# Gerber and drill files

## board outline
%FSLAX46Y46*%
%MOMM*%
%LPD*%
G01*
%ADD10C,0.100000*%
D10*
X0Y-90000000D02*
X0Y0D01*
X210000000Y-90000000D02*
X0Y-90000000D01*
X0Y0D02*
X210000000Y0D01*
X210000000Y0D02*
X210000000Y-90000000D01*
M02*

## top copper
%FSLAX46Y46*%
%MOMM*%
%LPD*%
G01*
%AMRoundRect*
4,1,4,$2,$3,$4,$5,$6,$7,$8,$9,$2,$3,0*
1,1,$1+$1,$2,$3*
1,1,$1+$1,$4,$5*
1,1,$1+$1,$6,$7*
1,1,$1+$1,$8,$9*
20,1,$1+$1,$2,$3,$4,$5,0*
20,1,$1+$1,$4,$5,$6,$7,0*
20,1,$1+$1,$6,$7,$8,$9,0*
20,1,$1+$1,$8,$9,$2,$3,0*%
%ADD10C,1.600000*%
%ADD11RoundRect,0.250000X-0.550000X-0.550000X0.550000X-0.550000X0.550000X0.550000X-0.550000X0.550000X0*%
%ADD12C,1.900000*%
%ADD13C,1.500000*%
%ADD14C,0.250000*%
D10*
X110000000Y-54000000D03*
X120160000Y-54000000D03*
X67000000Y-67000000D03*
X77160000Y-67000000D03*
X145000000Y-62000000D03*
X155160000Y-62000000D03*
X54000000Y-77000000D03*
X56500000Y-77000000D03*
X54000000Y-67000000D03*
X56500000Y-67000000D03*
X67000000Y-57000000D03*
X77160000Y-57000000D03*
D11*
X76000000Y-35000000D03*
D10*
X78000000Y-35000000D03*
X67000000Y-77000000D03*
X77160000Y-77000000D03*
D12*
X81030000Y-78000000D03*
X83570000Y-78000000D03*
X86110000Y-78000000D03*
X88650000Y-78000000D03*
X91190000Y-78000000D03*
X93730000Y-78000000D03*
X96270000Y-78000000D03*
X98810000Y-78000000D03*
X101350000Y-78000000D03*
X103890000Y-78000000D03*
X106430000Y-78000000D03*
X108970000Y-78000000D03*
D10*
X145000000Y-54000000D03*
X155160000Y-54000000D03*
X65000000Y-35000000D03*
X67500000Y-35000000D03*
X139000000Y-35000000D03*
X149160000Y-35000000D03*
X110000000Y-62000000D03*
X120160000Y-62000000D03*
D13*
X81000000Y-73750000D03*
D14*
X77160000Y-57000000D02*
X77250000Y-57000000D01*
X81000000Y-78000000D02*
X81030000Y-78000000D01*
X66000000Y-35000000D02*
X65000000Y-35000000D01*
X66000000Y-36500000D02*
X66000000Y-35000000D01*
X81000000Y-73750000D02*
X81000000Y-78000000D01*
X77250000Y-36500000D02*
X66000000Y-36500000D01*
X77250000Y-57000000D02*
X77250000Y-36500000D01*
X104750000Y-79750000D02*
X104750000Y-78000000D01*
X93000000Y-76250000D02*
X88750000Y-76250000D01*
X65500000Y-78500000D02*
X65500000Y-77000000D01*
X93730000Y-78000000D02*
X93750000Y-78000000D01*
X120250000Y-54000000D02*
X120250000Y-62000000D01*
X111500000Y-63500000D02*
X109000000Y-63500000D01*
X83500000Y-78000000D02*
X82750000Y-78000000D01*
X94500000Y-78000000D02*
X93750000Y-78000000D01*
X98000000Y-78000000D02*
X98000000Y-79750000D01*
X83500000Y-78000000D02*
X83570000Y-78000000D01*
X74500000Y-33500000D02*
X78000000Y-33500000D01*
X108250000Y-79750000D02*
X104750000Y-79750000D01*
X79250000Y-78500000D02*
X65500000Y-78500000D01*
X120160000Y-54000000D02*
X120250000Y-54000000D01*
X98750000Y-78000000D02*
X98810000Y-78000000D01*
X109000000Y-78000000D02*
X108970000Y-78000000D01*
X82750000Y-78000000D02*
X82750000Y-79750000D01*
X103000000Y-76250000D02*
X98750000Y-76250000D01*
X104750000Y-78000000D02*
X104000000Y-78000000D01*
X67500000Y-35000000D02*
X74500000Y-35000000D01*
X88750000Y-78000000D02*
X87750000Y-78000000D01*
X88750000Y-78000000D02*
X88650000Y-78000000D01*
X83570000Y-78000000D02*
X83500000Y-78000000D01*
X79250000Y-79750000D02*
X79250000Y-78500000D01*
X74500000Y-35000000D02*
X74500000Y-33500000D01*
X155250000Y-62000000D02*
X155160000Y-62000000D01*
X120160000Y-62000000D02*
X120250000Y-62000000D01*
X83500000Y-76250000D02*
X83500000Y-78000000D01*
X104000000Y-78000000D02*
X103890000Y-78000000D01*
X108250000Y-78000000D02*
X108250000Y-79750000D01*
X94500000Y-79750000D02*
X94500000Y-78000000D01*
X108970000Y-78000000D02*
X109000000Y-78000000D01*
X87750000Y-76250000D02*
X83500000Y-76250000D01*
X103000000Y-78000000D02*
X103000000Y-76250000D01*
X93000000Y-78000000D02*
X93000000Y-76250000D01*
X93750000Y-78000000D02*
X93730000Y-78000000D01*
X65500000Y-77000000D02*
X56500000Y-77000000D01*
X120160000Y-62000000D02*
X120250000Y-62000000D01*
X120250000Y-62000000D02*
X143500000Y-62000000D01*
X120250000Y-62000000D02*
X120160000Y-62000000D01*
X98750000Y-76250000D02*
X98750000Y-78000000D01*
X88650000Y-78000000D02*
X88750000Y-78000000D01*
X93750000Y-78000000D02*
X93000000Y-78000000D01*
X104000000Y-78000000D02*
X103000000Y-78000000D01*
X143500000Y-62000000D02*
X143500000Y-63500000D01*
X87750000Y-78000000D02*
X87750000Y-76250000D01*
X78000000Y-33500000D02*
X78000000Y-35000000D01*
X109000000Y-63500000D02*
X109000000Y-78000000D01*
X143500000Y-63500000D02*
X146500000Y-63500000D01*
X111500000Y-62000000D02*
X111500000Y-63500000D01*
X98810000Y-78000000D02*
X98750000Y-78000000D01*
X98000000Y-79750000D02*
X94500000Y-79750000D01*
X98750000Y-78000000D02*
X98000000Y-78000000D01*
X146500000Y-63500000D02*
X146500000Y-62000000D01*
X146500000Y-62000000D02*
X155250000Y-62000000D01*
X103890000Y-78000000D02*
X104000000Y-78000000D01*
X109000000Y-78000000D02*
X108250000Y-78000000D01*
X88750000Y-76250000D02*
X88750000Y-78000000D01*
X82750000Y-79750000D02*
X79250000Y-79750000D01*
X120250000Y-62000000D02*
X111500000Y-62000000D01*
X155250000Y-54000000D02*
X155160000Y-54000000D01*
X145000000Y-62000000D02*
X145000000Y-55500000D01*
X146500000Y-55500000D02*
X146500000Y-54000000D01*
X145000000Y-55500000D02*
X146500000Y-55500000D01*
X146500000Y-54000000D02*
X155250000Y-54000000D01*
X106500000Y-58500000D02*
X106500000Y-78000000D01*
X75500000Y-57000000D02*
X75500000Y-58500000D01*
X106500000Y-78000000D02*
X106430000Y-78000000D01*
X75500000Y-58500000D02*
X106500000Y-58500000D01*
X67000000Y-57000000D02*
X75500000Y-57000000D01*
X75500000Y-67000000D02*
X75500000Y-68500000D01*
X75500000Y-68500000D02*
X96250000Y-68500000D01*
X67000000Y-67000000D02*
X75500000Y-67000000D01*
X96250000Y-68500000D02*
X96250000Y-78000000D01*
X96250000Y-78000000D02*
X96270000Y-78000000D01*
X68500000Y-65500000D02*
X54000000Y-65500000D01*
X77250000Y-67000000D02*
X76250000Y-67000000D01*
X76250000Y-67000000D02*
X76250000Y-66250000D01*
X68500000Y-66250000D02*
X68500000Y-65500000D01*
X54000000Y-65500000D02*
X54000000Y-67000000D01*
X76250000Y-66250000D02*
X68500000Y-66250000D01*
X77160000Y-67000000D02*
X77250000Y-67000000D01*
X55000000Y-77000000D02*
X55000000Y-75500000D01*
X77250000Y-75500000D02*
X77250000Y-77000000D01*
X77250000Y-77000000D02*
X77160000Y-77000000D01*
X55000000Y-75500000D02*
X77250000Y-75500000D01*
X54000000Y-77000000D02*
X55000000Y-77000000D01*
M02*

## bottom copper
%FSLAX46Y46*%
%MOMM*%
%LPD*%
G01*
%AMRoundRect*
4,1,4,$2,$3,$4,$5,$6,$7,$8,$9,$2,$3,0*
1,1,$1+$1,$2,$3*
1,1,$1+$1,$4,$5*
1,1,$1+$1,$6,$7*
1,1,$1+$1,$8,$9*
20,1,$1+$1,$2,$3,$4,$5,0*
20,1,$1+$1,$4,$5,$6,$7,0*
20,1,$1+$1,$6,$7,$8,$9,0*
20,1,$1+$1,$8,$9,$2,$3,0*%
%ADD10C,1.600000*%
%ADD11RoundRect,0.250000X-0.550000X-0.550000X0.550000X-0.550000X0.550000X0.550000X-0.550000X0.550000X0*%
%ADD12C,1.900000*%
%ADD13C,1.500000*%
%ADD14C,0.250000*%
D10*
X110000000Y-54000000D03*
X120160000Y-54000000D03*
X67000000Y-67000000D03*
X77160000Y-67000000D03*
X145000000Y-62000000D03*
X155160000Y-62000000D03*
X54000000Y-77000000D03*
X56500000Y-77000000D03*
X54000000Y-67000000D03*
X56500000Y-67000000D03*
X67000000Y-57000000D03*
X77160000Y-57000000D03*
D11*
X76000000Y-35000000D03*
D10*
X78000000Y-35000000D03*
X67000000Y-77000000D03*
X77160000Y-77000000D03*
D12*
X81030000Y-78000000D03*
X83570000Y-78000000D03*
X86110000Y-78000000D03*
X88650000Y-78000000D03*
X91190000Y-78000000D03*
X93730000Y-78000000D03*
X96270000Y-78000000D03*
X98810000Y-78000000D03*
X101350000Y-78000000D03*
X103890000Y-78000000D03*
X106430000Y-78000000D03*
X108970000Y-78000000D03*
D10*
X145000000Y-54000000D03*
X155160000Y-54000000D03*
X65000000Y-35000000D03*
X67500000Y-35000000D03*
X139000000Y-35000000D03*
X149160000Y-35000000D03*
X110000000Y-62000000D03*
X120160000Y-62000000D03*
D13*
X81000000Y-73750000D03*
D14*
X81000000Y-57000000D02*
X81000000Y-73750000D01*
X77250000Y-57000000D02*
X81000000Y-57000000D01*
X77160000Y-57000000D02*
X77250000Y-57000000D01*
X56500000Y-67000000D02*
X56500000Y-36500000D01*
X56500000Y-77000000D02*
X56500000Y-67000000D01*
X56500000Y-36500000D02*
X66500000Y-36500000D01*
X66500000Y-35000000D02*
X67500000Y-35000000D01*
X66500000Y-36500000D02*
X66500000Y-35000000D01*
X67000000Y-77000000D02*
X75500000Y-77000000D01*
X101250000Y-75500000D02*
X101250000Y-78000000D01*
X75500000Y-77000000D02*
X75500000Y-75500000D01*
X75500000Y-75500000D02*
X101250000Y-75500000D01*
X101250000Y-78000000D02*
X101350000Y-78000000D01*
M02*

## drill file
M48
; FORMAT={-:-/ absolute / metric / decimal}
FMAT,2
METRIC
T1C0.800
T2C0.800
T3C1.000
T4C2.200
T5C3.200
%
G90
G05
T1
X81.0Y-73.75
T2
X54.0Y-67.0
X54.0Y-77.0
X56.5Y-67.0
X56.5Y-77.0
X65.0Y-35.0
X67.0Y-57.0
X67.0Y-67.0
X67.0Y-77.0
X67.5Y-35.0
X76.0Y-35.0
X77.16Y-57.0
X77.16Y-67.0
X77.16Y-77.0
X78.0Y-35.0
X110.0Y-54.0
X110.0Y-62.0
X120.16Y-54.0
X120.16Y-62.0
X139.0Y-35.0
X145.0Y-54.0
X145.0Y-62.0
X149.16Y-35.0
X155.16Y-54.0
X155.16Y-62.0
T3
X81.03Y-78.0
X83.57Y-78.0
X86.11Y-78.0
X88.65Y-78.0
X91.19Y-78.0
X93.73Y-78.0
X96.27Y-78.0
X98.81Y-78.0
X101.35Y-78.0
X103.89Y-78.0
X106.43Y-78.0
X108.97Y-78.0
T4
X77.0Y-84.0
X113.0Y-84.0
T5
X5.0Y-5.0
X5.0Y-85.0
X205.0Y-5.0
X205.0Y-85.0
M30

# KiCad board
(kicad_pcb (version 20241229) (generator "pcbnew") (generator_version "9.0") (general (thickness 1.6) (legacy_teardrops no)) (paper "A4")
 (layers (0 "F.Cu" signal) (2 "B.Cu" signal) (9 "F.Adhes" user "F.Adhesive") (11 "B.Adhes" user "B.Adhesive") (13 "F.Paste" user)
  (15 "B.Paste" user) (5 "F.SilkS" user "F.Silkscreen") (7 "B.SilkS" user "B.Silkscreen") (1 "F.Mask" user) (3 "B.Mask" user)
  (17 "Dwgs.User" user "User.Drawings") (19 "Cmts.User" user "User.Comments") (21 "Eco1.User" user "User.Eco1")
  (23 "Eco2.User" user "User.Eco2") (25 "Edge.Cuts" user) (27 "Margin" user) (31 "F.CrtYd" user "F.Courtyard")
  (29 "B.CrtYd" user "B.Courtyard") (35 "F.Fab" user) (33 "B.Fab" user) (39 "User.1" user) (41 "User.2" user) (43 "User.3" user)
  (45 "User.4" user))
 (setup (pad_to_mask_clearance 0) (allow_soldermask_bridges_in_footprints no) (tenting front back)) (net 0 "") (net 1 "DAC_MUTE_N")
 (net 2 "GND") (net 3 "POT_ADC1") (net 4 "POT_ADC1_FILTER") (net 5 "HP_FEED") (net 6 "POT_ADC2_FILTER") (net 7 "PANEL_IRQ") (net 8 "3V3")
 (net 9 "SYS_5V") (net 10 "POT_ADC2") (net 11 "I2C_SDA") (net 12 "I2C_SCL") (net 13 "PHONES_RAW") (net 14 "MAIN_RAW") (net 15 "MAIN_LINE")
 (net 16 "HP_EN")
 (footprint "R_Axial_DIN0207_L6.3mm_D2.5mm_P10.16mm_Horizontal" (layer "F.Cu") (at 110 54)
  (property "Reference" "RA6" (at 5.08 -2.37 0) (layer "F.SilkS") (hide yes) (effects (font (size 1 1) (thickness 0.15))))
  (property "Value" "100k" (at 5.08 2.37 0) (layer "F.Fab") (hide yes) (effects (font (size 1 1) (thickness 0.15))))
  (pad "1" thru_hole circle (at 0 0) (size 1.6 1.6) (drill 0.8) (layers "*.Cu" "*.Mask") (remove_unused_layers no) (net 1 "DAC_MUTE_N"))
  (pad "2" thru_hole circle (at 10.16 0) (size 1.6 1.6) (drill 0.8) (layers "*.Cu" "*.Mask") (remove_unused_layers no) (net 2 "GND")))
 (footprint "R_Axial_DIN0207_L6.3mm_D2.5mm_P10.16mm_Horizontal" (layer "F.Cu") (at 67 67)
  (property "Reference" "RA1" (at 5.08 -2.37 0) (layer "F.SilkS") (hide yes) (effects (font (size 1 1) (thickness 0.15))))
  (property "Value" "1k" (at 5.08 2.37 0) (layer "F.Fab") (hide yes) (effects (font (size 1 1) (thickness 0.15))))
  (pad "1" thru_hole circle (at 0 0) (size 1.6 1.6) (drill 0.8) (layers "*.Cu" "*.Mask") (remove_unused_layers no) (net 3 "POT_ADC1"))
  (pad "2" thru_hole circle (at 10.16 0) (size 1.6 1.6) (drill 0.8) (layers "*.Cu" "*.Mask") (remove_unused_layers no)
   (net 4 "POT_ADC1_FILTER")))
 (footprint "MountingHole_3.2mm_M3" (layer "F.Cu") (at 5 5)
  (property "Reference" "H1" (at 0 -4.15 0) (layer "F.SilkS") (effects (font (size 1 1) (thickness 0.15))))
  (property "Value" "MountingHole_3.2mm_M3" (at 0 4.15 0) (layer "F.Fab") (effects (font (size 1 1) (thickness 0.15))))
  (pad "" np_thru_hole circle (at 0 0) (size 3.2 3.2) (drill 3.2) (layers "*.Cu" "*.Mask")))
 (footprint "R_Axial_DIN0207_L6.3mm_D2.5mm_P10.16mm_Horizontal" (layer "F.Cu") (at 145 62)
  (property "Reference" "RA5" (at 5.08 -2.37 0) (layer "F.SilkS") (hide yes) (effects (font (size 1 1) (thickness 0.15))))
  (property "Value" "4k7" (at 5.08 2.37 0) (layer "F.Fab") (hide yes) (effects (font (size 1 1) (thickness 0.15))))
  (pad "1" thru_hole circle (at 0 0) (size 1.6 1.6) (drill 0.8) (layers "*.Cu" "*.Mask") (remove_unused_layers no) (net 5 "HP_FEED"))
  (pad "2" thru_hole circle (at 10.16 0) (size 1.6 1.6) (drill 0.8) (layers "*.Cu" "*.Mask") (remove_unused_layers no) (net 2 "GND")))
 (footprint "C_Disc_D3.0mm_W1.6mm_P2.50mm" (layer "F.Cu") (at 54 77)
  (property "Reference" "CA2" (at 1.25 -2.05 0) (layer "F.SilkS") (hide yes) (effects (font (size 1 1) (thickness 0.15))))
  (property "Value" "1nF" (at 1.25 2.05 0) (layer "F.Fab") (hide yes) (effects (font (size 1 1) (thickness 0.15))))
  (pad "1" thru_hole circle (at 0 0) (size 1.6 1.6) (drill 0.8) (layers "*.Cu" "*.Mask") (remove_unused_layers no) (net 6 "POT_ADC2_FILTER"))
  (pad "2" thru_hole circle (at 2.5 0) (size 1.6 1.6) (drill 0.8) (layers "*.Cu" "*.Mask") (remove_unused_layers no) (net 2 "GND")))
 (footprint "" (layer "F.Cu") (at 112 42)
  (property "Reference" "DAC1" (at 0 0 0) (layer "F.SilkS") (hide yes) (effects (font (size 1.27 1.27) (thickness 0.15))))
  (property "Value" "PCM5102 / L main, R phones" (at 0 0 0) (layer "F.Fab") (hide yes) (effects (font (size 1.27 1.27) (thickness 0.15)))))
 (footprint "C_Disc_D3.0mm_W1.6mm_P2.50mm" (layer "F.Cu") (at 54 67)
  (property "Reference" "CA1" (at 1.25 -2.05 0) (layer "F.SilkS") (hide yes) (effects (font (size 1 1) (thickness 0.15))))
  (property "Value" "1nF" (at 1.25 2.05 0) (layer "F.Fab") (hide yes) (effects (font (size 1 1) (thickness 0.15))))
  (pad "1" thru_hole circle (at 0 0) (size 1.6 1.6) (drill 0.8) (layers "*.Cu" "*.Mask") (remove_unused_layers no) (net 4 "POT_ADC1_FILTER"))
  (pad "2" thru_hole circle (at 2.5 0) (size 1.6 1.6) (drill 0.8) (layers "*.Cu" "*.Mask") (remove_unused_layers no) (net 2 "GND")))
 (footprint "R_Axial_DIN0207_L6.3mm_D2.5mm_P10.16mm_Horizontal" (layer "F.Cu") (at 67 57)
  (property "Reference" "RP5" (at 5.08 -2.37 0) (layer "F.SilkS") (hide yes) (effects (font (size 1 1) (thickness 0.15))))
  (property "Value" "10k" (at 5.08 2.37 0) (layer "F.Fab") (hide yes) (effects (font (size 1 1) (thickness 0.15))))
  (pad "1" thru_hole circle (at 0 0) (size 1.6 1.6) (drill 0.8) (layers "*.Cu" "*.Mask") (remove_unused_layers no) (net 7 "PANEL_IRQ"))
  (pad "2" thru_hole circle (at 10.16 0) (size 1.6 1.6) (drill 0.8) (layers "*.Cu" "*.Mask") (remove_unused_layers no) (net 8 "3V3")))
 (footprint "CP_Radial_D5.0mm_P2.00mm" (layer "F.Cu") (at 76 35)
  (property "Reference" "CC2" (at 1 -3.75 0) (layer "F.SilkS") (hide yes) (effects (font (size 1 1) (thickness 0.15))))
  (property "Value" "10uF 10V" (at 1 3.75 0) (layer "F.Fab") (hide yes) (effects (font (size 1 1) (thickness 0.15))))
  (pad "1" thru_hole roundrect (at 0 0) (size 1.6 1.6) (drill 0.8) (layers "*.Cu" "*.Mask") (remove_unused_layers no)
   (roundrect_rratio 0.15625) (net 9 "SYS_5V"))
  (pad "2" thru_hole circle (at 2 0) (size 1.6 1.6) (drill 0.8) (layers "*.Cu" "*.Mask") (remove_unused_layers no) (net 2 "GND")))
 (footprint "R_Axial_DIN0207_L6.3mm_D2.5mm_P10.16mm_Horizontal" (layer "F.Cu") (at 67 77)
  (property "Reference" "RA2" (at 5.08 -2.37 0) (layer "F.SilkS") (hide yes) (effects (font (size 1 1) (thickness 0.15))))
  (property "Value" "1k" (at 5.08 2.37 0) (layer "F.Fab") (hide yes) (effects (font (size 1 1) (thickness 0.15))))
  (pad "1" thru_hole circle (at 0 0) (size 1.6 1.6) (drill 0.8) (layers "*.Cu" "*.Mask") (remove_unused_layers no) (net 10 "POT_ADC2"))
  (pad "2" thru_hole circle (at 10.16 0) (size 1.6 1.6) (drill 0.8) (layers "*.Cu" "*.Mask") (remove_unused_layers no)
   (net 6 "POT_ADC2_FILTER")))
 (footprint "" (layer "F.Cu") (at 174 13)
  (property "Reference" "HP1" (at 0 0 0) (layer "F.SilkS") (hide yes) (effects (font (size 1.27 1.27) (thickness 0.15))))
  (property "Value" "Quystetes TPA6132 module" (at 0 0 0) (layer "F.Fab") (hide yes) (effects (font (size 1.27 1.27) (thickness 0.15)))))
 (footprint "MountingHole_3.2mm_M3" (layer "F.Cu") (at 205 5)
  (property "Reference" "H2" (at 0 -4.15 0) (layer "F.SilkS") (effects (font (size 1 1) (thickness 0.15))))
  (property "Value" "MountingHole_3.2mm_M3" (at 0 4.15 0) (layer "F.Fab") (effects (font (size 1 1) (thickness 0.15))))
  (pad "" np_thru_hole circle (at 0 0) (size 3.2 3.2) (drill 3.2) (layers "*.Cu" "*.Mask")))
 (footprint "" (layer "F.Cu") (at 95 78)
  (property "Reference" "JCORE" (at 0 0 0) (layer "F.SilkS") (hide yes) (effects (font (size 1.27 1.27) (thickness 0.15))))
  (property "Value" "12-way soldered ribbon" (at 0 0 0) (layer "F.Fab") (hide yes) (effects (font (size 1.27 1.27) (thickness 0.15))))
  (pad "1" thru_hole circle (at -13.97 0) (size 1.9 1.9) (drill 1) (layers "*.Cu") (remove_unused_layers no) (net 8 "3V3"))
  (pad "2" thru_hole circle (at -11.43 0) (size 1.9 1.9) (drill 1) (layers "*.Cu") (remove_unused_layers no) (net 2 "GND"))
  (pad "3" thru_hole circle (at -8.89 0) (size 1.9 1.9) (drill 1) (layers "*.Cu") (remove_unused_layers no) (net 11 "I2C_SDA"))
  (pad "4" thru_hole circle (at -6.35 0) (size 1.9 1.9) (drill 1) (layers "*.Cu") (remove_unused_layers no) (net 2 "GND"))
  (pad "5" thru_hole circle (at -3.81 0) (size 1.9 1.9) (drill 1) (layers "*.Cu") (remove_unused_layers no) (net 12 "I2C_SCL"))
  (pad "6" thru_hole circle (at -1.27 0) (size 1.9 1.9) (drill 1) (layers "*.Cu") (remove_unused_layers no) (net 2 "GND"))
  (pad "7" thru_hole circle (at 1.27 0) (size 1.9 1.9) (drill 1) (layers "*.Cu") (remove_unused_layers no) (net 3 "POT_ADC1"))
  (pad "8" thru_hole circle (at 3.81 0) (size 1.9 1.9) (drill 1) (layers "*.Cu") (remove_unused_layers no) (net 2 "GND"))
  (pad "9" thru_hole circle (at 6.35 0) (size 1.9 1.9) (drill 1) (layers "*.Cu") (remove_unused_layers no) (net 10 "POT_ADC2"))
  (pad "10" thru_hole circle (at 8.89 0) (size 1.9 1.9) (drill 1) (layers "*.Cu") (remove_unused_layers no) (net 2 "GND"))
  (pad "11" thru_hole circle (at 11.43 0) (size 1.9 1.9) (drill 1) (layers "*.Cu") (remove_unused_layers no) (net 7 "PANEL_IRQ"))
  (pad "12" thru_hole circle (at 13.97 0) (size 1.9 1.9) (drill 1) (layers "*.Cu") (remove_unused_layers no) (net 2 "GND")))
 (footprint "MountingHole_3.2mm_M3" (layer "F.Cu") (at 5 85)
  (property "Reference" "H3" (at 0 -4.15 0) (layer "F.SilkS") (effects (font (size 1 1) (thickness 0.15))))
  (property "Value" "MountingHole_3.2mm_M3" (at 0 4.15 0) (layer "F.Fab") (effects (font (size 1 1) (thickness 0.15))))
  (pad "" np_thru_hole circle (at 0 0) (size 3.2 3.2) (drill 3.2) (layers "*.Cu" "*.Mask")))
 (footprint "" (layer "F.Cu") (at 144 5)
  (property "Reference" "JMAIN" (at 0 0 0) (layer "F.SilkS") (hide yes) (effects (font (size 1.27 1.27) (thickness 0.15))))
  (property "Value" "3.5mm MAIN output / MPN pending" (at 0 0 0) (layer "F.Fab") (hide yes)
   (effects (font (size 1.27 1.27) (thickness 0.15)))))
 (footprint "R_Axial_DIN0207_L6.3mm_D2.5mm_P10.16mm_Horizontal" (layer "F.Cu") (at 145 54)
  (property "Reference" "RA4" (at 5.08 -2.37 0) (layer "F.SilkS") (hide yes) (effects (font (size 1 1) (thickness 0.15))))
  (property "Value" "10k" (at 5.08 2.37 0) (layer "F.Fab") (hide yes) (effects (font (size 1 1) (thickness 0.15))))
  (pad "1" thru_hole circle (at 0 0) (size 1.6 1.6) (drill 0.8) (layers "*.Cu" "*.Mask") (remove_unused_layers no) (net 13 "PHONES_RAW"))
  (pad "2" thru_hole circle (at 10.16 0) (size 1.6 1.6) (drill 0.8) (layers "*.Cu" "*.Mask") (remove_unused_layers no) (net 5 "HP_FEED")))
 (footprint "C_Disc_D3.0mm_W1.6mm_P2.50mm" (layer "F.Cu") (at 65 35)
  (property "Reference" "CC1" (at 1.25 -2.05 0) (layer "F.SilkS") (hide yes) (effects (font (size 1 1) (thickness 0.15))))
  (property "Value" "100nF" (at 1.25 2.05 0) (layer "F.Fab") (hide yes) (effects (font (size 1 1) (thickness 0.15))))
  (pad "1" thru_hole circle (at 0 0) (size 1.6 1.6) (drill 0.8) (layers "*.Cu" "*.Mask") (remove_unused_layers no) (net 8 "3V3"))
  (pad "2" thru_hole circle (at 2.5 0) (size 1.6 1.6) (drill 0.8) (layers "*.Cu" "*.Mask") (remove_unused_layers no) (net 2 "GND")))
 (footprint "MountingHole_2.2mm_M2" (layer "F.Cu") (at 77 84)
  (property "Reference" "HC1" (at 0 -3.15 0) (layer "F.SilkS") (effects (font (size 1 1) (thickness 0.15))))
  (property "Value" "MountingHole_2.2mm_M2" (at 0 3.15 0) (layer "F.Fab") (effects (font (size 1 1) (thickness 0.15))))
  (pad "" np_thru_hole circle (at 0 0) (size 2.2 2.2) (drill 2.2) (layers "*.Cu" "*.Mask")))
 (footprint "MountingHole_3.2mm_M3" (layer "F.Cu") (at 205 85)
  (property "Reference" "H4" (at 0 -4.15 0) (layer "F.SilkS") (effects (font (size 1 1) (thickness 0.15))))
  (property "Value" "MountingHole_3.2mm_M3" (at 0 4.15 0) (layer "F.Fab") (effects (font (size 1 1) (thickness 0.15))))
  (pad "" np_thru_hole circle (at 0 0) (size 3.2 3.2) (drill 3.2) (layers "*.Cu" "*.Mask")))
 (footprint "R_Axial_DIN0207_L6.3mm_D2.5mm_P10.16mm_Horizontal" (layer "F.Cu") (at 139 35)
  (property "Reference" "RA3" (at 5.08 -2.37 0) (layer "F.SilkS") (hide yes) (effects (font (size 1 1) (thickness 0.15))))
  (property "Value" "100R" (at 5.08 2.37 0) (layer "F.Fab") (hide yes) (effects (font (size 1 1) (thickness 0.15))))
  (pad "1" thru_hole circle (at 0 0) (size 1.6 1.6) (drill 0.8) (layers "*.Cu" "*.Mask") (remove_unused_layers no) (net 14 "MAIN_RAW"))
  (pad "2" thru_hole circle (at 10.16 0) (size 1.6 1.6) (drill 0.8) (layers "*.Cu" "*.Mask") (remove_unused_layers no) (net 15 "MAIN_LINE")))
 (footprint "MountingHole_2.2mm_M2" (layer "F.Cu") (at 113 84)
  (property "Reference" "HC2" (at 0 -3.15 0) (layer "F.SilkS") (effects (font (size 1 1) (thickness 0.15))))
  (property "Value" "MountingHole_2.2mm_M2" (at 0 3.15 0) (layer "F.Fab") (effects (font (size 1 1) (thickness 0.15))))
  (pad "" np_thru_hole circle (at 0 0) (size 2.2 2.2) (drill 2.2) (layers "*.Cu" "*.Mask")))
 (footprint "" (layer "F.Cu") (at 30 31)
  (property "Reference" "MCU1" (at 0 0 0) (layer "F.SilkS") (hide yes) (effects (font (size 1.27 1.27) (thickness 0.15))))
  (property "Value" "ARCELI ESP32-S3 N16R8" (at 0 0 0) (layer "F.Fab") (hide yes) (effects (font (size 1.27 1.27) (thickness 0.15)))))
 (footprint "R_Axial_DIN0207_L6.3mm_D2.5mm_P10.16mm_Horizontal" (layer "F.Cu") (at 110 62)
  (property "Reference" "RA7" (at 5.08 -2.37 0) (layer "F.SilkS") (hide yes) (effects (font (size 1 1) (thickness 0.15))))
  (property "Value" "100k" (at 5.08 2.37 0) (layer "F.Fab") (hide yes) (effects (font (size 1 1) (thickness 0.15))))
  (pad "1" thru_hole circle (at 0 0) (size 1.6 1.6) (drill 0.8) (layers "*.Cu" "*.Mask") (remove_unused_layers no) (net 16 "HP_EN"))
  (pad "2" thru_hole circle (at 10.16 0) (size 1.6 1.6) (drill 0.8) (layers "*.Cu" "*.Mask") (remove_unused_layers no) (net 2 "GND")))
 (gr_line (start 0 90) (end 0 0) (stroke (width 0.1) (type default)) (layer "Edge.Cuts"))
 (gr_line (start 210 90) (end 0 90) (stroke (width 0.1) (type default)) (layer "Edge.Cuts"))
 (gr_line (start 0 0) (end 210 0) (stroke (width 0.1) (type default)) (layer "Edge.Cuts"))
 (gr_line (start 210 0) (end 210 90) (stroke (width 0.1) (type default)) (layer "Edge.Cuts"))
 (segment (start 77.16 57) (end 77.25 57) (width 0.25) (layer "F.Cu") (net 8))
 (segment (start 81 78) (end 81.03 78) (width 0.25) (layer "F.Cu") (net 8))
 (segment (start 66 35) (end 65 35) (width 0.25) (layer "F.Cu") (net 8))
 (segment (start 66 36.5) (end 66 35) (width 0.25) (layer "F.Cu") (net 8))
 (segment (start 81 73.75) (end 81 78) (width 0.25) (layer "F.Cu") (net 8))
 (segment (start 77.25 36.5) (end 66 36.5) (width 0.25) (layer "F.Cu") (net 8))
 (segment (start 77.25 57) (end 77.25 36.5) (width 0.25) (layer "F.Cu") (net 8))
 (via (at 81 73.75) (size 1.5) (drill 0.8) (layers "F.Cu" "B.Cu") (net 8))
 (segment (start 81 57) (end 81 73.75) (width 0.25) (layer "B.Cu") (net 8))
 (segment (start 77.25 57) (end 81 57) (width 0.25) (layer "B.Cu") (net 8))
 (segment (start 77.16 57) (end 77.25 57) (width 0.25) (layer "B.Cu") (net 8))
 (segment (start 104.75 79.75) (end 104.75 78) (width 0.25) (layer "F.Cu") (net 2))
 (segment (start 93 76.25) (end 88.75 76.25) (width 0.25) (layer "F.Cu") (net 2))
 (segment (start 65.5 78.5) (end 65.5 77) (width 0.25) (layer "F.Cu") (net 2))
 (segment (start 93.73 78) (end 93.75 78) (width 0.25) (layer "F.Cu") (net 2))
 (segment (start 120.25 54) (end 120.25 62) (width 0.25) (layer "F.Cu") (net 2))
 (segment (start 111.5 63.5) (end 109 63.5) (width 0.25) (layer "F.Cu") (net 2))
 (segment (start 83.5 78) (end 82.75 78) (width 0.25) (layer "F.Cu") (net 2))
 (segment (start 94.5 78) (end 93.75 78) (width 0.25) (layer "F.Cu") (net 2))
 (segment (start 98 78) (end 98 79.75) (width 0.25) (layer "F.Cu") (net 2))
 (segment (start 83.5 78) (end 83.57 78) (width 0.25) (layer "F.Cu") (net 2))
 (segment (start 74.5 33.5) (end 78 33.5) (width 0.25) (layer "F.Cu") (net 2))
 (segment (start 108.25 79.75) (end 104.75 79.75) (width 0.25) (layer "F.Cu") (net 2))
 (segment (start 79.25 78.5) (end 65.5 78.5) (width 0.25) (layer "F.Cu") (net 2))
 (segment (start 120.16 54) (end 120.25 54) (width 0.25) (layer "F.Cu") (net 2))
 (segment (start 98.75 78) (end 98.81 78) (width 0.25) (layer "F.Cu") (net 2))
 (segment (start 109 78) (end 108.97 78) (width 0.25) (layer "F.Cu") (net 2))
 (segment (start 82.75 78) (end 82.75 79.75) (width 0.25) (layer "F.Cu") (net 2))
 (segment (start 103 76.25) (end 98.75 76.25) (width 0.25) (layer "F.Cu") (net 2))
 (segment (start 104.75 78) (end 104 78) (width 0.25) (layer "F.Cu") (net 2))
 (segment (start 67.5 35) (end 74.5 35) (width 0.25) (layer "F.Cu") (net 2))
 (segment (start 88.75 78) (end 87.75 78) (width 0.25) (layer "F.Cu") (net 2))
 (segment (start 88.75 78) (end 88.65 78) (width 0.25) (layer "F.Cu") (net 2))
 (segment (start 83.57 78) (end 83.5 78) (width 0.25) (layer "F.Cu") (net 2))
 (segment (start 79.25 79.75) (end 79.25 78.5) (width 0.25) (layer "F.Cu") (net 2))
 (segment (start 74.5 35) (end 74.5 33.5) (width 0.25) (layer "F.Cu") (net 2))
 (segment (start 155.25 62) (end 155.16 62) (width 0.25) (layer "F.Cu") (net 2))
 (segment (start 120.16 62) (end 120.25 62) (width 0.25) (layer "F.Cu") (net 2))
 (segment (start 83.5 76.25) (end 83.5 78) (width 0.25) (layer "F.Cu") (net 2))
 (segment (start 104 78) (end 103.89 78) (width 0.25) (layer "F.Cu") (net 2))
 (segment (start 108.25 78) (end 108.25 79.75) (width 0.25) (layer "F.Cu") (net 2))
 (segment (start 94.5 79.75) (end 94.5 78) (width 0.25) (layer "F.Cu") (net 2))
 (segment (start 108.97 78) (end 109 78) (width 0.25) (layer "F.Cu") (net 2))
 (segment (start 87.75 76.25) (end 83.5 76.25) (width 0.25) (layer "F.Cu") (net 2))
 (segment (start 103 78) (end 103 76.25) (width 0.25) (layer "F.Cu") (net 2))
 (segment (start 93 78) (end 93 76.25) (width 0.25) (layer "F.Cu") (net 2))
 (segment (start 93.75 78) (end 93.73 78) (width 0.25) (layer "F.Cu") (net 2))
 (segment (start 65.5 77) (end 56.5 77) (width 0.25) (layer "F.Cu") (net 2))
 (segment (start 120.16 62) (end 120.25 62) (width 0.25) (layer "F.Cu") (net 2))
 (segment (start 120.25 62) (end 143.5 62) (width 0.25) (layer "F.Cu") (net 2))
 (segment (start 120.25 62) (end 120.16 62) (width 0.25) (layer "F.Cu") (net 2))
 (segment (start 98.75 76.25) (end 98.75 78) (width 0.25) (layer "F.Cu") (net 2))
 (segment (start 88.65 78) (end 88.75 78) (width 0.25) (layer "F.Cu") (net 2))
 (segment (start 93.75 78) (end 93 78) (width 0.25) (layer "F.Cu") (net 2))
 (segment (start 104 78) (end 103 78) (width 0.25) (layer "F.Cu") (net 2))
 (segment (start 143.5 62) (end 143.5 63.5) (width 0.25) (layer "F.Cu") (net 2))
 (segment (start 87.75 78) (end 87.75 76.25) (width 0.25) (layer "F.Cu") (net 2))
 (segment (start 78 33.5) (end 78 35) (width 0.25) (layer "F.Cu") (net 2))
 (segment (start 109 63.5) (end 109 78) (width 0.25) (layer "F.Cu") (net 2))
 (segment (start 143.5 63.5) (end 146.5 63.5) (width 0.25) (layer "F.Cu") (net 2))
 (segment (start 111.5 62) (end 111.5 63.5) (width 0.25) (layer "F.Cu") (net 2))
 (segment (start 98.81 78) (end 98.75 78) (width 0.25) (layer "F.Cu") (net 2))
 (segment (start 98 79.75) (end 94.5 79.75) (width 0.25) (layer "F.Cu") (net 2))
 (segment (start 98.75 78) (end 98 78) (width 0.25) (layer "F.Cu") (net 2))
 (segment (start 146.5 63.5) (end 146.5 62) (width 0.25) (layer "F.Cu") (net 2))
 (segment (start 146.5 62) (end 155.25 62) (width 0.25) (layer "F.Cu") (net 2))
 (segment (start 103.89 78) (end 104 78) (width 0.25) (layer "F.Cu") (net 2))
 (segment (start 109 78) (end 108.25 78) (width 0.25) (layer "F.Cu") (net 2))
 (segment (start 88.75 76.25) (end 88.75 78) (width 0.25) (layer "F.Cu") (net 2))
 (segment (start 82.75 79.75) (end 79.25 79.75) (width 0.25) (layer "F.Cu") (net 2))
 (segment (start 120.25 62) (end 111.5 62) (width 0.25) (layer "F.Cu") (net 2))
 (segment (start 56.5 67) (end 56.5 36.5) (width 0.25) (layer "B.Cu") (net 2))
 (segment (start 56.5 77) (end 56.5 67) (width 0.25) (layer "B.Cu") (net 2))
 (segment (start 56.5 36.5) (end 66.5 36.5) (width 0.25) (layer "B.Cu") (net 2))
 (segment (start 66.5 35) (end 67.5 35) (width 0.25) (layer "B.Cu") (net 2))
 (segment (start 66.5 36.5) (end 66.5 35) (width 0.25) (layer "B.Cu") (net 2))
 (segment (start 155.25 54) (end 155.16 54) (width 0.25) (layer "F.Cu") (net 5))
 (segment (start 145 62) (end 145 55.5) (width 0.25) (layer "F.Cu") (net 5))
 (segment (start 146.5 55.5) (end 146.5 54) (width 0.25) (layer "F.Cu") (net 5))
 (segment (start 145 55.5) (end 146.5 55.5) (width 0.25) (layer "F.Cu") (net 5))
 (segment (start 146.5 54) (end 155.25 54) (width 0.25) (layer "F.Cu") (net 5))
 (segment (start 106.5 58.5) (end 106.5 78) (width 0.25) (layer "F.Cu") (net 7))
 (segment (start 75.5 57) (end 75.5 58.5) (width 0.25) (layer "F.Cu") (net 7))
 (segment (start 106.5 78) (end 106.43 78) (width 0.25) (layer "F.Cu") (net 7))
 (segment (start 75.5 58.5) (end 106.5 58.5) (width 0.25) (layer "F.Cu") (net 7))
 (segment (start 67 57) (end 75.5 57) (width 0.25) (layer "F.Cu") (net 7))
 (segment (start 75.5 67) (end 75.5 68.5) (width 0.25) (layer "F.Cu") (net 3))
 (segment (start 75.5 68.5) (end 96.25 68.5) (width 0.25) (layer "F.Cu") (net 3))
 (segment (start 67 67) (end 75.5 67) (width 0.25) (layer "F.Cu") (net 3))
 (segment (start 96.25 68.5) (end 96.25 78) (width 0.25) (layer "F.Cu") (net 3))
 (segment (start 96.25 78) (end 96.27 78) (width 0.25) (layer "F.Cu") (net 3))
 (segment (start 68.5 65.5) (end 54 65.5) (width 0.25) (layer "F.Cu") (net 4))
 (segment (start 77.25 67) (end 76.25 67) (width 0.25) (layer "F.Cu") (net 4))
 (segment (start 76.25 67) (end 76.25 66.25) (width 0.25) (layer "F.Cu") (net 4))
 (segment (start 68.5 66.25) (end 68.5 65.5) (width 0.25) (layer "F.Cu") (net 4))
 (segment (start 54 65.5) (end 54 67) (width 0.25) (layer "F.Cu") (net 4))
 (segment (start 76.25 66.25) (end 68.5 66.25) (width 0.25) (layer "F.Cu") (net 4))
 (segment (start 77.16 67) (end 77.25 67) (width 0.25) (layer "F.Cu") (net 4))
 (segment (start 67 77) (end 75.5 77) (width 0.25) (layer "B.Cu") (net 10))
 (segment (start 101.25 75.5) (end 101.25 78) (width 0.25) (layer "B.Cu") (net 10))
 (segment (start 75.5 77) (end 75.5 75.5) (width 0.25) (layer "B.Cu") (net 10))
 (segment (start 75.5 75.5) (end 101.25 75.5) (width 0.25) (layer "B.Cu") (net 10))
 (segment (start 101.25 78) (end 101.35 78) (width 0.25) (layer "B.Cu") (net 10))
 (segment (start 55 77) (end 55 75.5) (width 0.25) (layer "F.Cu") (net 6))
 (segment (start 77.25 75.5) (end 77.25 77) (width 0.25) (layer "F.Cu") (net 6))
 (segment (start 77.25 77) (end 77.16 77) (width 0.25) (layer "F.Cu") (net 6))
 (segment (start 55 75.5) (end 77.25 75.5) (width 0.25) (layer "F.Cu") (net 6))
 (segment (start 54 77) (end 55 77) (width 0.25) (layer "F.Cu") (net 6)))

